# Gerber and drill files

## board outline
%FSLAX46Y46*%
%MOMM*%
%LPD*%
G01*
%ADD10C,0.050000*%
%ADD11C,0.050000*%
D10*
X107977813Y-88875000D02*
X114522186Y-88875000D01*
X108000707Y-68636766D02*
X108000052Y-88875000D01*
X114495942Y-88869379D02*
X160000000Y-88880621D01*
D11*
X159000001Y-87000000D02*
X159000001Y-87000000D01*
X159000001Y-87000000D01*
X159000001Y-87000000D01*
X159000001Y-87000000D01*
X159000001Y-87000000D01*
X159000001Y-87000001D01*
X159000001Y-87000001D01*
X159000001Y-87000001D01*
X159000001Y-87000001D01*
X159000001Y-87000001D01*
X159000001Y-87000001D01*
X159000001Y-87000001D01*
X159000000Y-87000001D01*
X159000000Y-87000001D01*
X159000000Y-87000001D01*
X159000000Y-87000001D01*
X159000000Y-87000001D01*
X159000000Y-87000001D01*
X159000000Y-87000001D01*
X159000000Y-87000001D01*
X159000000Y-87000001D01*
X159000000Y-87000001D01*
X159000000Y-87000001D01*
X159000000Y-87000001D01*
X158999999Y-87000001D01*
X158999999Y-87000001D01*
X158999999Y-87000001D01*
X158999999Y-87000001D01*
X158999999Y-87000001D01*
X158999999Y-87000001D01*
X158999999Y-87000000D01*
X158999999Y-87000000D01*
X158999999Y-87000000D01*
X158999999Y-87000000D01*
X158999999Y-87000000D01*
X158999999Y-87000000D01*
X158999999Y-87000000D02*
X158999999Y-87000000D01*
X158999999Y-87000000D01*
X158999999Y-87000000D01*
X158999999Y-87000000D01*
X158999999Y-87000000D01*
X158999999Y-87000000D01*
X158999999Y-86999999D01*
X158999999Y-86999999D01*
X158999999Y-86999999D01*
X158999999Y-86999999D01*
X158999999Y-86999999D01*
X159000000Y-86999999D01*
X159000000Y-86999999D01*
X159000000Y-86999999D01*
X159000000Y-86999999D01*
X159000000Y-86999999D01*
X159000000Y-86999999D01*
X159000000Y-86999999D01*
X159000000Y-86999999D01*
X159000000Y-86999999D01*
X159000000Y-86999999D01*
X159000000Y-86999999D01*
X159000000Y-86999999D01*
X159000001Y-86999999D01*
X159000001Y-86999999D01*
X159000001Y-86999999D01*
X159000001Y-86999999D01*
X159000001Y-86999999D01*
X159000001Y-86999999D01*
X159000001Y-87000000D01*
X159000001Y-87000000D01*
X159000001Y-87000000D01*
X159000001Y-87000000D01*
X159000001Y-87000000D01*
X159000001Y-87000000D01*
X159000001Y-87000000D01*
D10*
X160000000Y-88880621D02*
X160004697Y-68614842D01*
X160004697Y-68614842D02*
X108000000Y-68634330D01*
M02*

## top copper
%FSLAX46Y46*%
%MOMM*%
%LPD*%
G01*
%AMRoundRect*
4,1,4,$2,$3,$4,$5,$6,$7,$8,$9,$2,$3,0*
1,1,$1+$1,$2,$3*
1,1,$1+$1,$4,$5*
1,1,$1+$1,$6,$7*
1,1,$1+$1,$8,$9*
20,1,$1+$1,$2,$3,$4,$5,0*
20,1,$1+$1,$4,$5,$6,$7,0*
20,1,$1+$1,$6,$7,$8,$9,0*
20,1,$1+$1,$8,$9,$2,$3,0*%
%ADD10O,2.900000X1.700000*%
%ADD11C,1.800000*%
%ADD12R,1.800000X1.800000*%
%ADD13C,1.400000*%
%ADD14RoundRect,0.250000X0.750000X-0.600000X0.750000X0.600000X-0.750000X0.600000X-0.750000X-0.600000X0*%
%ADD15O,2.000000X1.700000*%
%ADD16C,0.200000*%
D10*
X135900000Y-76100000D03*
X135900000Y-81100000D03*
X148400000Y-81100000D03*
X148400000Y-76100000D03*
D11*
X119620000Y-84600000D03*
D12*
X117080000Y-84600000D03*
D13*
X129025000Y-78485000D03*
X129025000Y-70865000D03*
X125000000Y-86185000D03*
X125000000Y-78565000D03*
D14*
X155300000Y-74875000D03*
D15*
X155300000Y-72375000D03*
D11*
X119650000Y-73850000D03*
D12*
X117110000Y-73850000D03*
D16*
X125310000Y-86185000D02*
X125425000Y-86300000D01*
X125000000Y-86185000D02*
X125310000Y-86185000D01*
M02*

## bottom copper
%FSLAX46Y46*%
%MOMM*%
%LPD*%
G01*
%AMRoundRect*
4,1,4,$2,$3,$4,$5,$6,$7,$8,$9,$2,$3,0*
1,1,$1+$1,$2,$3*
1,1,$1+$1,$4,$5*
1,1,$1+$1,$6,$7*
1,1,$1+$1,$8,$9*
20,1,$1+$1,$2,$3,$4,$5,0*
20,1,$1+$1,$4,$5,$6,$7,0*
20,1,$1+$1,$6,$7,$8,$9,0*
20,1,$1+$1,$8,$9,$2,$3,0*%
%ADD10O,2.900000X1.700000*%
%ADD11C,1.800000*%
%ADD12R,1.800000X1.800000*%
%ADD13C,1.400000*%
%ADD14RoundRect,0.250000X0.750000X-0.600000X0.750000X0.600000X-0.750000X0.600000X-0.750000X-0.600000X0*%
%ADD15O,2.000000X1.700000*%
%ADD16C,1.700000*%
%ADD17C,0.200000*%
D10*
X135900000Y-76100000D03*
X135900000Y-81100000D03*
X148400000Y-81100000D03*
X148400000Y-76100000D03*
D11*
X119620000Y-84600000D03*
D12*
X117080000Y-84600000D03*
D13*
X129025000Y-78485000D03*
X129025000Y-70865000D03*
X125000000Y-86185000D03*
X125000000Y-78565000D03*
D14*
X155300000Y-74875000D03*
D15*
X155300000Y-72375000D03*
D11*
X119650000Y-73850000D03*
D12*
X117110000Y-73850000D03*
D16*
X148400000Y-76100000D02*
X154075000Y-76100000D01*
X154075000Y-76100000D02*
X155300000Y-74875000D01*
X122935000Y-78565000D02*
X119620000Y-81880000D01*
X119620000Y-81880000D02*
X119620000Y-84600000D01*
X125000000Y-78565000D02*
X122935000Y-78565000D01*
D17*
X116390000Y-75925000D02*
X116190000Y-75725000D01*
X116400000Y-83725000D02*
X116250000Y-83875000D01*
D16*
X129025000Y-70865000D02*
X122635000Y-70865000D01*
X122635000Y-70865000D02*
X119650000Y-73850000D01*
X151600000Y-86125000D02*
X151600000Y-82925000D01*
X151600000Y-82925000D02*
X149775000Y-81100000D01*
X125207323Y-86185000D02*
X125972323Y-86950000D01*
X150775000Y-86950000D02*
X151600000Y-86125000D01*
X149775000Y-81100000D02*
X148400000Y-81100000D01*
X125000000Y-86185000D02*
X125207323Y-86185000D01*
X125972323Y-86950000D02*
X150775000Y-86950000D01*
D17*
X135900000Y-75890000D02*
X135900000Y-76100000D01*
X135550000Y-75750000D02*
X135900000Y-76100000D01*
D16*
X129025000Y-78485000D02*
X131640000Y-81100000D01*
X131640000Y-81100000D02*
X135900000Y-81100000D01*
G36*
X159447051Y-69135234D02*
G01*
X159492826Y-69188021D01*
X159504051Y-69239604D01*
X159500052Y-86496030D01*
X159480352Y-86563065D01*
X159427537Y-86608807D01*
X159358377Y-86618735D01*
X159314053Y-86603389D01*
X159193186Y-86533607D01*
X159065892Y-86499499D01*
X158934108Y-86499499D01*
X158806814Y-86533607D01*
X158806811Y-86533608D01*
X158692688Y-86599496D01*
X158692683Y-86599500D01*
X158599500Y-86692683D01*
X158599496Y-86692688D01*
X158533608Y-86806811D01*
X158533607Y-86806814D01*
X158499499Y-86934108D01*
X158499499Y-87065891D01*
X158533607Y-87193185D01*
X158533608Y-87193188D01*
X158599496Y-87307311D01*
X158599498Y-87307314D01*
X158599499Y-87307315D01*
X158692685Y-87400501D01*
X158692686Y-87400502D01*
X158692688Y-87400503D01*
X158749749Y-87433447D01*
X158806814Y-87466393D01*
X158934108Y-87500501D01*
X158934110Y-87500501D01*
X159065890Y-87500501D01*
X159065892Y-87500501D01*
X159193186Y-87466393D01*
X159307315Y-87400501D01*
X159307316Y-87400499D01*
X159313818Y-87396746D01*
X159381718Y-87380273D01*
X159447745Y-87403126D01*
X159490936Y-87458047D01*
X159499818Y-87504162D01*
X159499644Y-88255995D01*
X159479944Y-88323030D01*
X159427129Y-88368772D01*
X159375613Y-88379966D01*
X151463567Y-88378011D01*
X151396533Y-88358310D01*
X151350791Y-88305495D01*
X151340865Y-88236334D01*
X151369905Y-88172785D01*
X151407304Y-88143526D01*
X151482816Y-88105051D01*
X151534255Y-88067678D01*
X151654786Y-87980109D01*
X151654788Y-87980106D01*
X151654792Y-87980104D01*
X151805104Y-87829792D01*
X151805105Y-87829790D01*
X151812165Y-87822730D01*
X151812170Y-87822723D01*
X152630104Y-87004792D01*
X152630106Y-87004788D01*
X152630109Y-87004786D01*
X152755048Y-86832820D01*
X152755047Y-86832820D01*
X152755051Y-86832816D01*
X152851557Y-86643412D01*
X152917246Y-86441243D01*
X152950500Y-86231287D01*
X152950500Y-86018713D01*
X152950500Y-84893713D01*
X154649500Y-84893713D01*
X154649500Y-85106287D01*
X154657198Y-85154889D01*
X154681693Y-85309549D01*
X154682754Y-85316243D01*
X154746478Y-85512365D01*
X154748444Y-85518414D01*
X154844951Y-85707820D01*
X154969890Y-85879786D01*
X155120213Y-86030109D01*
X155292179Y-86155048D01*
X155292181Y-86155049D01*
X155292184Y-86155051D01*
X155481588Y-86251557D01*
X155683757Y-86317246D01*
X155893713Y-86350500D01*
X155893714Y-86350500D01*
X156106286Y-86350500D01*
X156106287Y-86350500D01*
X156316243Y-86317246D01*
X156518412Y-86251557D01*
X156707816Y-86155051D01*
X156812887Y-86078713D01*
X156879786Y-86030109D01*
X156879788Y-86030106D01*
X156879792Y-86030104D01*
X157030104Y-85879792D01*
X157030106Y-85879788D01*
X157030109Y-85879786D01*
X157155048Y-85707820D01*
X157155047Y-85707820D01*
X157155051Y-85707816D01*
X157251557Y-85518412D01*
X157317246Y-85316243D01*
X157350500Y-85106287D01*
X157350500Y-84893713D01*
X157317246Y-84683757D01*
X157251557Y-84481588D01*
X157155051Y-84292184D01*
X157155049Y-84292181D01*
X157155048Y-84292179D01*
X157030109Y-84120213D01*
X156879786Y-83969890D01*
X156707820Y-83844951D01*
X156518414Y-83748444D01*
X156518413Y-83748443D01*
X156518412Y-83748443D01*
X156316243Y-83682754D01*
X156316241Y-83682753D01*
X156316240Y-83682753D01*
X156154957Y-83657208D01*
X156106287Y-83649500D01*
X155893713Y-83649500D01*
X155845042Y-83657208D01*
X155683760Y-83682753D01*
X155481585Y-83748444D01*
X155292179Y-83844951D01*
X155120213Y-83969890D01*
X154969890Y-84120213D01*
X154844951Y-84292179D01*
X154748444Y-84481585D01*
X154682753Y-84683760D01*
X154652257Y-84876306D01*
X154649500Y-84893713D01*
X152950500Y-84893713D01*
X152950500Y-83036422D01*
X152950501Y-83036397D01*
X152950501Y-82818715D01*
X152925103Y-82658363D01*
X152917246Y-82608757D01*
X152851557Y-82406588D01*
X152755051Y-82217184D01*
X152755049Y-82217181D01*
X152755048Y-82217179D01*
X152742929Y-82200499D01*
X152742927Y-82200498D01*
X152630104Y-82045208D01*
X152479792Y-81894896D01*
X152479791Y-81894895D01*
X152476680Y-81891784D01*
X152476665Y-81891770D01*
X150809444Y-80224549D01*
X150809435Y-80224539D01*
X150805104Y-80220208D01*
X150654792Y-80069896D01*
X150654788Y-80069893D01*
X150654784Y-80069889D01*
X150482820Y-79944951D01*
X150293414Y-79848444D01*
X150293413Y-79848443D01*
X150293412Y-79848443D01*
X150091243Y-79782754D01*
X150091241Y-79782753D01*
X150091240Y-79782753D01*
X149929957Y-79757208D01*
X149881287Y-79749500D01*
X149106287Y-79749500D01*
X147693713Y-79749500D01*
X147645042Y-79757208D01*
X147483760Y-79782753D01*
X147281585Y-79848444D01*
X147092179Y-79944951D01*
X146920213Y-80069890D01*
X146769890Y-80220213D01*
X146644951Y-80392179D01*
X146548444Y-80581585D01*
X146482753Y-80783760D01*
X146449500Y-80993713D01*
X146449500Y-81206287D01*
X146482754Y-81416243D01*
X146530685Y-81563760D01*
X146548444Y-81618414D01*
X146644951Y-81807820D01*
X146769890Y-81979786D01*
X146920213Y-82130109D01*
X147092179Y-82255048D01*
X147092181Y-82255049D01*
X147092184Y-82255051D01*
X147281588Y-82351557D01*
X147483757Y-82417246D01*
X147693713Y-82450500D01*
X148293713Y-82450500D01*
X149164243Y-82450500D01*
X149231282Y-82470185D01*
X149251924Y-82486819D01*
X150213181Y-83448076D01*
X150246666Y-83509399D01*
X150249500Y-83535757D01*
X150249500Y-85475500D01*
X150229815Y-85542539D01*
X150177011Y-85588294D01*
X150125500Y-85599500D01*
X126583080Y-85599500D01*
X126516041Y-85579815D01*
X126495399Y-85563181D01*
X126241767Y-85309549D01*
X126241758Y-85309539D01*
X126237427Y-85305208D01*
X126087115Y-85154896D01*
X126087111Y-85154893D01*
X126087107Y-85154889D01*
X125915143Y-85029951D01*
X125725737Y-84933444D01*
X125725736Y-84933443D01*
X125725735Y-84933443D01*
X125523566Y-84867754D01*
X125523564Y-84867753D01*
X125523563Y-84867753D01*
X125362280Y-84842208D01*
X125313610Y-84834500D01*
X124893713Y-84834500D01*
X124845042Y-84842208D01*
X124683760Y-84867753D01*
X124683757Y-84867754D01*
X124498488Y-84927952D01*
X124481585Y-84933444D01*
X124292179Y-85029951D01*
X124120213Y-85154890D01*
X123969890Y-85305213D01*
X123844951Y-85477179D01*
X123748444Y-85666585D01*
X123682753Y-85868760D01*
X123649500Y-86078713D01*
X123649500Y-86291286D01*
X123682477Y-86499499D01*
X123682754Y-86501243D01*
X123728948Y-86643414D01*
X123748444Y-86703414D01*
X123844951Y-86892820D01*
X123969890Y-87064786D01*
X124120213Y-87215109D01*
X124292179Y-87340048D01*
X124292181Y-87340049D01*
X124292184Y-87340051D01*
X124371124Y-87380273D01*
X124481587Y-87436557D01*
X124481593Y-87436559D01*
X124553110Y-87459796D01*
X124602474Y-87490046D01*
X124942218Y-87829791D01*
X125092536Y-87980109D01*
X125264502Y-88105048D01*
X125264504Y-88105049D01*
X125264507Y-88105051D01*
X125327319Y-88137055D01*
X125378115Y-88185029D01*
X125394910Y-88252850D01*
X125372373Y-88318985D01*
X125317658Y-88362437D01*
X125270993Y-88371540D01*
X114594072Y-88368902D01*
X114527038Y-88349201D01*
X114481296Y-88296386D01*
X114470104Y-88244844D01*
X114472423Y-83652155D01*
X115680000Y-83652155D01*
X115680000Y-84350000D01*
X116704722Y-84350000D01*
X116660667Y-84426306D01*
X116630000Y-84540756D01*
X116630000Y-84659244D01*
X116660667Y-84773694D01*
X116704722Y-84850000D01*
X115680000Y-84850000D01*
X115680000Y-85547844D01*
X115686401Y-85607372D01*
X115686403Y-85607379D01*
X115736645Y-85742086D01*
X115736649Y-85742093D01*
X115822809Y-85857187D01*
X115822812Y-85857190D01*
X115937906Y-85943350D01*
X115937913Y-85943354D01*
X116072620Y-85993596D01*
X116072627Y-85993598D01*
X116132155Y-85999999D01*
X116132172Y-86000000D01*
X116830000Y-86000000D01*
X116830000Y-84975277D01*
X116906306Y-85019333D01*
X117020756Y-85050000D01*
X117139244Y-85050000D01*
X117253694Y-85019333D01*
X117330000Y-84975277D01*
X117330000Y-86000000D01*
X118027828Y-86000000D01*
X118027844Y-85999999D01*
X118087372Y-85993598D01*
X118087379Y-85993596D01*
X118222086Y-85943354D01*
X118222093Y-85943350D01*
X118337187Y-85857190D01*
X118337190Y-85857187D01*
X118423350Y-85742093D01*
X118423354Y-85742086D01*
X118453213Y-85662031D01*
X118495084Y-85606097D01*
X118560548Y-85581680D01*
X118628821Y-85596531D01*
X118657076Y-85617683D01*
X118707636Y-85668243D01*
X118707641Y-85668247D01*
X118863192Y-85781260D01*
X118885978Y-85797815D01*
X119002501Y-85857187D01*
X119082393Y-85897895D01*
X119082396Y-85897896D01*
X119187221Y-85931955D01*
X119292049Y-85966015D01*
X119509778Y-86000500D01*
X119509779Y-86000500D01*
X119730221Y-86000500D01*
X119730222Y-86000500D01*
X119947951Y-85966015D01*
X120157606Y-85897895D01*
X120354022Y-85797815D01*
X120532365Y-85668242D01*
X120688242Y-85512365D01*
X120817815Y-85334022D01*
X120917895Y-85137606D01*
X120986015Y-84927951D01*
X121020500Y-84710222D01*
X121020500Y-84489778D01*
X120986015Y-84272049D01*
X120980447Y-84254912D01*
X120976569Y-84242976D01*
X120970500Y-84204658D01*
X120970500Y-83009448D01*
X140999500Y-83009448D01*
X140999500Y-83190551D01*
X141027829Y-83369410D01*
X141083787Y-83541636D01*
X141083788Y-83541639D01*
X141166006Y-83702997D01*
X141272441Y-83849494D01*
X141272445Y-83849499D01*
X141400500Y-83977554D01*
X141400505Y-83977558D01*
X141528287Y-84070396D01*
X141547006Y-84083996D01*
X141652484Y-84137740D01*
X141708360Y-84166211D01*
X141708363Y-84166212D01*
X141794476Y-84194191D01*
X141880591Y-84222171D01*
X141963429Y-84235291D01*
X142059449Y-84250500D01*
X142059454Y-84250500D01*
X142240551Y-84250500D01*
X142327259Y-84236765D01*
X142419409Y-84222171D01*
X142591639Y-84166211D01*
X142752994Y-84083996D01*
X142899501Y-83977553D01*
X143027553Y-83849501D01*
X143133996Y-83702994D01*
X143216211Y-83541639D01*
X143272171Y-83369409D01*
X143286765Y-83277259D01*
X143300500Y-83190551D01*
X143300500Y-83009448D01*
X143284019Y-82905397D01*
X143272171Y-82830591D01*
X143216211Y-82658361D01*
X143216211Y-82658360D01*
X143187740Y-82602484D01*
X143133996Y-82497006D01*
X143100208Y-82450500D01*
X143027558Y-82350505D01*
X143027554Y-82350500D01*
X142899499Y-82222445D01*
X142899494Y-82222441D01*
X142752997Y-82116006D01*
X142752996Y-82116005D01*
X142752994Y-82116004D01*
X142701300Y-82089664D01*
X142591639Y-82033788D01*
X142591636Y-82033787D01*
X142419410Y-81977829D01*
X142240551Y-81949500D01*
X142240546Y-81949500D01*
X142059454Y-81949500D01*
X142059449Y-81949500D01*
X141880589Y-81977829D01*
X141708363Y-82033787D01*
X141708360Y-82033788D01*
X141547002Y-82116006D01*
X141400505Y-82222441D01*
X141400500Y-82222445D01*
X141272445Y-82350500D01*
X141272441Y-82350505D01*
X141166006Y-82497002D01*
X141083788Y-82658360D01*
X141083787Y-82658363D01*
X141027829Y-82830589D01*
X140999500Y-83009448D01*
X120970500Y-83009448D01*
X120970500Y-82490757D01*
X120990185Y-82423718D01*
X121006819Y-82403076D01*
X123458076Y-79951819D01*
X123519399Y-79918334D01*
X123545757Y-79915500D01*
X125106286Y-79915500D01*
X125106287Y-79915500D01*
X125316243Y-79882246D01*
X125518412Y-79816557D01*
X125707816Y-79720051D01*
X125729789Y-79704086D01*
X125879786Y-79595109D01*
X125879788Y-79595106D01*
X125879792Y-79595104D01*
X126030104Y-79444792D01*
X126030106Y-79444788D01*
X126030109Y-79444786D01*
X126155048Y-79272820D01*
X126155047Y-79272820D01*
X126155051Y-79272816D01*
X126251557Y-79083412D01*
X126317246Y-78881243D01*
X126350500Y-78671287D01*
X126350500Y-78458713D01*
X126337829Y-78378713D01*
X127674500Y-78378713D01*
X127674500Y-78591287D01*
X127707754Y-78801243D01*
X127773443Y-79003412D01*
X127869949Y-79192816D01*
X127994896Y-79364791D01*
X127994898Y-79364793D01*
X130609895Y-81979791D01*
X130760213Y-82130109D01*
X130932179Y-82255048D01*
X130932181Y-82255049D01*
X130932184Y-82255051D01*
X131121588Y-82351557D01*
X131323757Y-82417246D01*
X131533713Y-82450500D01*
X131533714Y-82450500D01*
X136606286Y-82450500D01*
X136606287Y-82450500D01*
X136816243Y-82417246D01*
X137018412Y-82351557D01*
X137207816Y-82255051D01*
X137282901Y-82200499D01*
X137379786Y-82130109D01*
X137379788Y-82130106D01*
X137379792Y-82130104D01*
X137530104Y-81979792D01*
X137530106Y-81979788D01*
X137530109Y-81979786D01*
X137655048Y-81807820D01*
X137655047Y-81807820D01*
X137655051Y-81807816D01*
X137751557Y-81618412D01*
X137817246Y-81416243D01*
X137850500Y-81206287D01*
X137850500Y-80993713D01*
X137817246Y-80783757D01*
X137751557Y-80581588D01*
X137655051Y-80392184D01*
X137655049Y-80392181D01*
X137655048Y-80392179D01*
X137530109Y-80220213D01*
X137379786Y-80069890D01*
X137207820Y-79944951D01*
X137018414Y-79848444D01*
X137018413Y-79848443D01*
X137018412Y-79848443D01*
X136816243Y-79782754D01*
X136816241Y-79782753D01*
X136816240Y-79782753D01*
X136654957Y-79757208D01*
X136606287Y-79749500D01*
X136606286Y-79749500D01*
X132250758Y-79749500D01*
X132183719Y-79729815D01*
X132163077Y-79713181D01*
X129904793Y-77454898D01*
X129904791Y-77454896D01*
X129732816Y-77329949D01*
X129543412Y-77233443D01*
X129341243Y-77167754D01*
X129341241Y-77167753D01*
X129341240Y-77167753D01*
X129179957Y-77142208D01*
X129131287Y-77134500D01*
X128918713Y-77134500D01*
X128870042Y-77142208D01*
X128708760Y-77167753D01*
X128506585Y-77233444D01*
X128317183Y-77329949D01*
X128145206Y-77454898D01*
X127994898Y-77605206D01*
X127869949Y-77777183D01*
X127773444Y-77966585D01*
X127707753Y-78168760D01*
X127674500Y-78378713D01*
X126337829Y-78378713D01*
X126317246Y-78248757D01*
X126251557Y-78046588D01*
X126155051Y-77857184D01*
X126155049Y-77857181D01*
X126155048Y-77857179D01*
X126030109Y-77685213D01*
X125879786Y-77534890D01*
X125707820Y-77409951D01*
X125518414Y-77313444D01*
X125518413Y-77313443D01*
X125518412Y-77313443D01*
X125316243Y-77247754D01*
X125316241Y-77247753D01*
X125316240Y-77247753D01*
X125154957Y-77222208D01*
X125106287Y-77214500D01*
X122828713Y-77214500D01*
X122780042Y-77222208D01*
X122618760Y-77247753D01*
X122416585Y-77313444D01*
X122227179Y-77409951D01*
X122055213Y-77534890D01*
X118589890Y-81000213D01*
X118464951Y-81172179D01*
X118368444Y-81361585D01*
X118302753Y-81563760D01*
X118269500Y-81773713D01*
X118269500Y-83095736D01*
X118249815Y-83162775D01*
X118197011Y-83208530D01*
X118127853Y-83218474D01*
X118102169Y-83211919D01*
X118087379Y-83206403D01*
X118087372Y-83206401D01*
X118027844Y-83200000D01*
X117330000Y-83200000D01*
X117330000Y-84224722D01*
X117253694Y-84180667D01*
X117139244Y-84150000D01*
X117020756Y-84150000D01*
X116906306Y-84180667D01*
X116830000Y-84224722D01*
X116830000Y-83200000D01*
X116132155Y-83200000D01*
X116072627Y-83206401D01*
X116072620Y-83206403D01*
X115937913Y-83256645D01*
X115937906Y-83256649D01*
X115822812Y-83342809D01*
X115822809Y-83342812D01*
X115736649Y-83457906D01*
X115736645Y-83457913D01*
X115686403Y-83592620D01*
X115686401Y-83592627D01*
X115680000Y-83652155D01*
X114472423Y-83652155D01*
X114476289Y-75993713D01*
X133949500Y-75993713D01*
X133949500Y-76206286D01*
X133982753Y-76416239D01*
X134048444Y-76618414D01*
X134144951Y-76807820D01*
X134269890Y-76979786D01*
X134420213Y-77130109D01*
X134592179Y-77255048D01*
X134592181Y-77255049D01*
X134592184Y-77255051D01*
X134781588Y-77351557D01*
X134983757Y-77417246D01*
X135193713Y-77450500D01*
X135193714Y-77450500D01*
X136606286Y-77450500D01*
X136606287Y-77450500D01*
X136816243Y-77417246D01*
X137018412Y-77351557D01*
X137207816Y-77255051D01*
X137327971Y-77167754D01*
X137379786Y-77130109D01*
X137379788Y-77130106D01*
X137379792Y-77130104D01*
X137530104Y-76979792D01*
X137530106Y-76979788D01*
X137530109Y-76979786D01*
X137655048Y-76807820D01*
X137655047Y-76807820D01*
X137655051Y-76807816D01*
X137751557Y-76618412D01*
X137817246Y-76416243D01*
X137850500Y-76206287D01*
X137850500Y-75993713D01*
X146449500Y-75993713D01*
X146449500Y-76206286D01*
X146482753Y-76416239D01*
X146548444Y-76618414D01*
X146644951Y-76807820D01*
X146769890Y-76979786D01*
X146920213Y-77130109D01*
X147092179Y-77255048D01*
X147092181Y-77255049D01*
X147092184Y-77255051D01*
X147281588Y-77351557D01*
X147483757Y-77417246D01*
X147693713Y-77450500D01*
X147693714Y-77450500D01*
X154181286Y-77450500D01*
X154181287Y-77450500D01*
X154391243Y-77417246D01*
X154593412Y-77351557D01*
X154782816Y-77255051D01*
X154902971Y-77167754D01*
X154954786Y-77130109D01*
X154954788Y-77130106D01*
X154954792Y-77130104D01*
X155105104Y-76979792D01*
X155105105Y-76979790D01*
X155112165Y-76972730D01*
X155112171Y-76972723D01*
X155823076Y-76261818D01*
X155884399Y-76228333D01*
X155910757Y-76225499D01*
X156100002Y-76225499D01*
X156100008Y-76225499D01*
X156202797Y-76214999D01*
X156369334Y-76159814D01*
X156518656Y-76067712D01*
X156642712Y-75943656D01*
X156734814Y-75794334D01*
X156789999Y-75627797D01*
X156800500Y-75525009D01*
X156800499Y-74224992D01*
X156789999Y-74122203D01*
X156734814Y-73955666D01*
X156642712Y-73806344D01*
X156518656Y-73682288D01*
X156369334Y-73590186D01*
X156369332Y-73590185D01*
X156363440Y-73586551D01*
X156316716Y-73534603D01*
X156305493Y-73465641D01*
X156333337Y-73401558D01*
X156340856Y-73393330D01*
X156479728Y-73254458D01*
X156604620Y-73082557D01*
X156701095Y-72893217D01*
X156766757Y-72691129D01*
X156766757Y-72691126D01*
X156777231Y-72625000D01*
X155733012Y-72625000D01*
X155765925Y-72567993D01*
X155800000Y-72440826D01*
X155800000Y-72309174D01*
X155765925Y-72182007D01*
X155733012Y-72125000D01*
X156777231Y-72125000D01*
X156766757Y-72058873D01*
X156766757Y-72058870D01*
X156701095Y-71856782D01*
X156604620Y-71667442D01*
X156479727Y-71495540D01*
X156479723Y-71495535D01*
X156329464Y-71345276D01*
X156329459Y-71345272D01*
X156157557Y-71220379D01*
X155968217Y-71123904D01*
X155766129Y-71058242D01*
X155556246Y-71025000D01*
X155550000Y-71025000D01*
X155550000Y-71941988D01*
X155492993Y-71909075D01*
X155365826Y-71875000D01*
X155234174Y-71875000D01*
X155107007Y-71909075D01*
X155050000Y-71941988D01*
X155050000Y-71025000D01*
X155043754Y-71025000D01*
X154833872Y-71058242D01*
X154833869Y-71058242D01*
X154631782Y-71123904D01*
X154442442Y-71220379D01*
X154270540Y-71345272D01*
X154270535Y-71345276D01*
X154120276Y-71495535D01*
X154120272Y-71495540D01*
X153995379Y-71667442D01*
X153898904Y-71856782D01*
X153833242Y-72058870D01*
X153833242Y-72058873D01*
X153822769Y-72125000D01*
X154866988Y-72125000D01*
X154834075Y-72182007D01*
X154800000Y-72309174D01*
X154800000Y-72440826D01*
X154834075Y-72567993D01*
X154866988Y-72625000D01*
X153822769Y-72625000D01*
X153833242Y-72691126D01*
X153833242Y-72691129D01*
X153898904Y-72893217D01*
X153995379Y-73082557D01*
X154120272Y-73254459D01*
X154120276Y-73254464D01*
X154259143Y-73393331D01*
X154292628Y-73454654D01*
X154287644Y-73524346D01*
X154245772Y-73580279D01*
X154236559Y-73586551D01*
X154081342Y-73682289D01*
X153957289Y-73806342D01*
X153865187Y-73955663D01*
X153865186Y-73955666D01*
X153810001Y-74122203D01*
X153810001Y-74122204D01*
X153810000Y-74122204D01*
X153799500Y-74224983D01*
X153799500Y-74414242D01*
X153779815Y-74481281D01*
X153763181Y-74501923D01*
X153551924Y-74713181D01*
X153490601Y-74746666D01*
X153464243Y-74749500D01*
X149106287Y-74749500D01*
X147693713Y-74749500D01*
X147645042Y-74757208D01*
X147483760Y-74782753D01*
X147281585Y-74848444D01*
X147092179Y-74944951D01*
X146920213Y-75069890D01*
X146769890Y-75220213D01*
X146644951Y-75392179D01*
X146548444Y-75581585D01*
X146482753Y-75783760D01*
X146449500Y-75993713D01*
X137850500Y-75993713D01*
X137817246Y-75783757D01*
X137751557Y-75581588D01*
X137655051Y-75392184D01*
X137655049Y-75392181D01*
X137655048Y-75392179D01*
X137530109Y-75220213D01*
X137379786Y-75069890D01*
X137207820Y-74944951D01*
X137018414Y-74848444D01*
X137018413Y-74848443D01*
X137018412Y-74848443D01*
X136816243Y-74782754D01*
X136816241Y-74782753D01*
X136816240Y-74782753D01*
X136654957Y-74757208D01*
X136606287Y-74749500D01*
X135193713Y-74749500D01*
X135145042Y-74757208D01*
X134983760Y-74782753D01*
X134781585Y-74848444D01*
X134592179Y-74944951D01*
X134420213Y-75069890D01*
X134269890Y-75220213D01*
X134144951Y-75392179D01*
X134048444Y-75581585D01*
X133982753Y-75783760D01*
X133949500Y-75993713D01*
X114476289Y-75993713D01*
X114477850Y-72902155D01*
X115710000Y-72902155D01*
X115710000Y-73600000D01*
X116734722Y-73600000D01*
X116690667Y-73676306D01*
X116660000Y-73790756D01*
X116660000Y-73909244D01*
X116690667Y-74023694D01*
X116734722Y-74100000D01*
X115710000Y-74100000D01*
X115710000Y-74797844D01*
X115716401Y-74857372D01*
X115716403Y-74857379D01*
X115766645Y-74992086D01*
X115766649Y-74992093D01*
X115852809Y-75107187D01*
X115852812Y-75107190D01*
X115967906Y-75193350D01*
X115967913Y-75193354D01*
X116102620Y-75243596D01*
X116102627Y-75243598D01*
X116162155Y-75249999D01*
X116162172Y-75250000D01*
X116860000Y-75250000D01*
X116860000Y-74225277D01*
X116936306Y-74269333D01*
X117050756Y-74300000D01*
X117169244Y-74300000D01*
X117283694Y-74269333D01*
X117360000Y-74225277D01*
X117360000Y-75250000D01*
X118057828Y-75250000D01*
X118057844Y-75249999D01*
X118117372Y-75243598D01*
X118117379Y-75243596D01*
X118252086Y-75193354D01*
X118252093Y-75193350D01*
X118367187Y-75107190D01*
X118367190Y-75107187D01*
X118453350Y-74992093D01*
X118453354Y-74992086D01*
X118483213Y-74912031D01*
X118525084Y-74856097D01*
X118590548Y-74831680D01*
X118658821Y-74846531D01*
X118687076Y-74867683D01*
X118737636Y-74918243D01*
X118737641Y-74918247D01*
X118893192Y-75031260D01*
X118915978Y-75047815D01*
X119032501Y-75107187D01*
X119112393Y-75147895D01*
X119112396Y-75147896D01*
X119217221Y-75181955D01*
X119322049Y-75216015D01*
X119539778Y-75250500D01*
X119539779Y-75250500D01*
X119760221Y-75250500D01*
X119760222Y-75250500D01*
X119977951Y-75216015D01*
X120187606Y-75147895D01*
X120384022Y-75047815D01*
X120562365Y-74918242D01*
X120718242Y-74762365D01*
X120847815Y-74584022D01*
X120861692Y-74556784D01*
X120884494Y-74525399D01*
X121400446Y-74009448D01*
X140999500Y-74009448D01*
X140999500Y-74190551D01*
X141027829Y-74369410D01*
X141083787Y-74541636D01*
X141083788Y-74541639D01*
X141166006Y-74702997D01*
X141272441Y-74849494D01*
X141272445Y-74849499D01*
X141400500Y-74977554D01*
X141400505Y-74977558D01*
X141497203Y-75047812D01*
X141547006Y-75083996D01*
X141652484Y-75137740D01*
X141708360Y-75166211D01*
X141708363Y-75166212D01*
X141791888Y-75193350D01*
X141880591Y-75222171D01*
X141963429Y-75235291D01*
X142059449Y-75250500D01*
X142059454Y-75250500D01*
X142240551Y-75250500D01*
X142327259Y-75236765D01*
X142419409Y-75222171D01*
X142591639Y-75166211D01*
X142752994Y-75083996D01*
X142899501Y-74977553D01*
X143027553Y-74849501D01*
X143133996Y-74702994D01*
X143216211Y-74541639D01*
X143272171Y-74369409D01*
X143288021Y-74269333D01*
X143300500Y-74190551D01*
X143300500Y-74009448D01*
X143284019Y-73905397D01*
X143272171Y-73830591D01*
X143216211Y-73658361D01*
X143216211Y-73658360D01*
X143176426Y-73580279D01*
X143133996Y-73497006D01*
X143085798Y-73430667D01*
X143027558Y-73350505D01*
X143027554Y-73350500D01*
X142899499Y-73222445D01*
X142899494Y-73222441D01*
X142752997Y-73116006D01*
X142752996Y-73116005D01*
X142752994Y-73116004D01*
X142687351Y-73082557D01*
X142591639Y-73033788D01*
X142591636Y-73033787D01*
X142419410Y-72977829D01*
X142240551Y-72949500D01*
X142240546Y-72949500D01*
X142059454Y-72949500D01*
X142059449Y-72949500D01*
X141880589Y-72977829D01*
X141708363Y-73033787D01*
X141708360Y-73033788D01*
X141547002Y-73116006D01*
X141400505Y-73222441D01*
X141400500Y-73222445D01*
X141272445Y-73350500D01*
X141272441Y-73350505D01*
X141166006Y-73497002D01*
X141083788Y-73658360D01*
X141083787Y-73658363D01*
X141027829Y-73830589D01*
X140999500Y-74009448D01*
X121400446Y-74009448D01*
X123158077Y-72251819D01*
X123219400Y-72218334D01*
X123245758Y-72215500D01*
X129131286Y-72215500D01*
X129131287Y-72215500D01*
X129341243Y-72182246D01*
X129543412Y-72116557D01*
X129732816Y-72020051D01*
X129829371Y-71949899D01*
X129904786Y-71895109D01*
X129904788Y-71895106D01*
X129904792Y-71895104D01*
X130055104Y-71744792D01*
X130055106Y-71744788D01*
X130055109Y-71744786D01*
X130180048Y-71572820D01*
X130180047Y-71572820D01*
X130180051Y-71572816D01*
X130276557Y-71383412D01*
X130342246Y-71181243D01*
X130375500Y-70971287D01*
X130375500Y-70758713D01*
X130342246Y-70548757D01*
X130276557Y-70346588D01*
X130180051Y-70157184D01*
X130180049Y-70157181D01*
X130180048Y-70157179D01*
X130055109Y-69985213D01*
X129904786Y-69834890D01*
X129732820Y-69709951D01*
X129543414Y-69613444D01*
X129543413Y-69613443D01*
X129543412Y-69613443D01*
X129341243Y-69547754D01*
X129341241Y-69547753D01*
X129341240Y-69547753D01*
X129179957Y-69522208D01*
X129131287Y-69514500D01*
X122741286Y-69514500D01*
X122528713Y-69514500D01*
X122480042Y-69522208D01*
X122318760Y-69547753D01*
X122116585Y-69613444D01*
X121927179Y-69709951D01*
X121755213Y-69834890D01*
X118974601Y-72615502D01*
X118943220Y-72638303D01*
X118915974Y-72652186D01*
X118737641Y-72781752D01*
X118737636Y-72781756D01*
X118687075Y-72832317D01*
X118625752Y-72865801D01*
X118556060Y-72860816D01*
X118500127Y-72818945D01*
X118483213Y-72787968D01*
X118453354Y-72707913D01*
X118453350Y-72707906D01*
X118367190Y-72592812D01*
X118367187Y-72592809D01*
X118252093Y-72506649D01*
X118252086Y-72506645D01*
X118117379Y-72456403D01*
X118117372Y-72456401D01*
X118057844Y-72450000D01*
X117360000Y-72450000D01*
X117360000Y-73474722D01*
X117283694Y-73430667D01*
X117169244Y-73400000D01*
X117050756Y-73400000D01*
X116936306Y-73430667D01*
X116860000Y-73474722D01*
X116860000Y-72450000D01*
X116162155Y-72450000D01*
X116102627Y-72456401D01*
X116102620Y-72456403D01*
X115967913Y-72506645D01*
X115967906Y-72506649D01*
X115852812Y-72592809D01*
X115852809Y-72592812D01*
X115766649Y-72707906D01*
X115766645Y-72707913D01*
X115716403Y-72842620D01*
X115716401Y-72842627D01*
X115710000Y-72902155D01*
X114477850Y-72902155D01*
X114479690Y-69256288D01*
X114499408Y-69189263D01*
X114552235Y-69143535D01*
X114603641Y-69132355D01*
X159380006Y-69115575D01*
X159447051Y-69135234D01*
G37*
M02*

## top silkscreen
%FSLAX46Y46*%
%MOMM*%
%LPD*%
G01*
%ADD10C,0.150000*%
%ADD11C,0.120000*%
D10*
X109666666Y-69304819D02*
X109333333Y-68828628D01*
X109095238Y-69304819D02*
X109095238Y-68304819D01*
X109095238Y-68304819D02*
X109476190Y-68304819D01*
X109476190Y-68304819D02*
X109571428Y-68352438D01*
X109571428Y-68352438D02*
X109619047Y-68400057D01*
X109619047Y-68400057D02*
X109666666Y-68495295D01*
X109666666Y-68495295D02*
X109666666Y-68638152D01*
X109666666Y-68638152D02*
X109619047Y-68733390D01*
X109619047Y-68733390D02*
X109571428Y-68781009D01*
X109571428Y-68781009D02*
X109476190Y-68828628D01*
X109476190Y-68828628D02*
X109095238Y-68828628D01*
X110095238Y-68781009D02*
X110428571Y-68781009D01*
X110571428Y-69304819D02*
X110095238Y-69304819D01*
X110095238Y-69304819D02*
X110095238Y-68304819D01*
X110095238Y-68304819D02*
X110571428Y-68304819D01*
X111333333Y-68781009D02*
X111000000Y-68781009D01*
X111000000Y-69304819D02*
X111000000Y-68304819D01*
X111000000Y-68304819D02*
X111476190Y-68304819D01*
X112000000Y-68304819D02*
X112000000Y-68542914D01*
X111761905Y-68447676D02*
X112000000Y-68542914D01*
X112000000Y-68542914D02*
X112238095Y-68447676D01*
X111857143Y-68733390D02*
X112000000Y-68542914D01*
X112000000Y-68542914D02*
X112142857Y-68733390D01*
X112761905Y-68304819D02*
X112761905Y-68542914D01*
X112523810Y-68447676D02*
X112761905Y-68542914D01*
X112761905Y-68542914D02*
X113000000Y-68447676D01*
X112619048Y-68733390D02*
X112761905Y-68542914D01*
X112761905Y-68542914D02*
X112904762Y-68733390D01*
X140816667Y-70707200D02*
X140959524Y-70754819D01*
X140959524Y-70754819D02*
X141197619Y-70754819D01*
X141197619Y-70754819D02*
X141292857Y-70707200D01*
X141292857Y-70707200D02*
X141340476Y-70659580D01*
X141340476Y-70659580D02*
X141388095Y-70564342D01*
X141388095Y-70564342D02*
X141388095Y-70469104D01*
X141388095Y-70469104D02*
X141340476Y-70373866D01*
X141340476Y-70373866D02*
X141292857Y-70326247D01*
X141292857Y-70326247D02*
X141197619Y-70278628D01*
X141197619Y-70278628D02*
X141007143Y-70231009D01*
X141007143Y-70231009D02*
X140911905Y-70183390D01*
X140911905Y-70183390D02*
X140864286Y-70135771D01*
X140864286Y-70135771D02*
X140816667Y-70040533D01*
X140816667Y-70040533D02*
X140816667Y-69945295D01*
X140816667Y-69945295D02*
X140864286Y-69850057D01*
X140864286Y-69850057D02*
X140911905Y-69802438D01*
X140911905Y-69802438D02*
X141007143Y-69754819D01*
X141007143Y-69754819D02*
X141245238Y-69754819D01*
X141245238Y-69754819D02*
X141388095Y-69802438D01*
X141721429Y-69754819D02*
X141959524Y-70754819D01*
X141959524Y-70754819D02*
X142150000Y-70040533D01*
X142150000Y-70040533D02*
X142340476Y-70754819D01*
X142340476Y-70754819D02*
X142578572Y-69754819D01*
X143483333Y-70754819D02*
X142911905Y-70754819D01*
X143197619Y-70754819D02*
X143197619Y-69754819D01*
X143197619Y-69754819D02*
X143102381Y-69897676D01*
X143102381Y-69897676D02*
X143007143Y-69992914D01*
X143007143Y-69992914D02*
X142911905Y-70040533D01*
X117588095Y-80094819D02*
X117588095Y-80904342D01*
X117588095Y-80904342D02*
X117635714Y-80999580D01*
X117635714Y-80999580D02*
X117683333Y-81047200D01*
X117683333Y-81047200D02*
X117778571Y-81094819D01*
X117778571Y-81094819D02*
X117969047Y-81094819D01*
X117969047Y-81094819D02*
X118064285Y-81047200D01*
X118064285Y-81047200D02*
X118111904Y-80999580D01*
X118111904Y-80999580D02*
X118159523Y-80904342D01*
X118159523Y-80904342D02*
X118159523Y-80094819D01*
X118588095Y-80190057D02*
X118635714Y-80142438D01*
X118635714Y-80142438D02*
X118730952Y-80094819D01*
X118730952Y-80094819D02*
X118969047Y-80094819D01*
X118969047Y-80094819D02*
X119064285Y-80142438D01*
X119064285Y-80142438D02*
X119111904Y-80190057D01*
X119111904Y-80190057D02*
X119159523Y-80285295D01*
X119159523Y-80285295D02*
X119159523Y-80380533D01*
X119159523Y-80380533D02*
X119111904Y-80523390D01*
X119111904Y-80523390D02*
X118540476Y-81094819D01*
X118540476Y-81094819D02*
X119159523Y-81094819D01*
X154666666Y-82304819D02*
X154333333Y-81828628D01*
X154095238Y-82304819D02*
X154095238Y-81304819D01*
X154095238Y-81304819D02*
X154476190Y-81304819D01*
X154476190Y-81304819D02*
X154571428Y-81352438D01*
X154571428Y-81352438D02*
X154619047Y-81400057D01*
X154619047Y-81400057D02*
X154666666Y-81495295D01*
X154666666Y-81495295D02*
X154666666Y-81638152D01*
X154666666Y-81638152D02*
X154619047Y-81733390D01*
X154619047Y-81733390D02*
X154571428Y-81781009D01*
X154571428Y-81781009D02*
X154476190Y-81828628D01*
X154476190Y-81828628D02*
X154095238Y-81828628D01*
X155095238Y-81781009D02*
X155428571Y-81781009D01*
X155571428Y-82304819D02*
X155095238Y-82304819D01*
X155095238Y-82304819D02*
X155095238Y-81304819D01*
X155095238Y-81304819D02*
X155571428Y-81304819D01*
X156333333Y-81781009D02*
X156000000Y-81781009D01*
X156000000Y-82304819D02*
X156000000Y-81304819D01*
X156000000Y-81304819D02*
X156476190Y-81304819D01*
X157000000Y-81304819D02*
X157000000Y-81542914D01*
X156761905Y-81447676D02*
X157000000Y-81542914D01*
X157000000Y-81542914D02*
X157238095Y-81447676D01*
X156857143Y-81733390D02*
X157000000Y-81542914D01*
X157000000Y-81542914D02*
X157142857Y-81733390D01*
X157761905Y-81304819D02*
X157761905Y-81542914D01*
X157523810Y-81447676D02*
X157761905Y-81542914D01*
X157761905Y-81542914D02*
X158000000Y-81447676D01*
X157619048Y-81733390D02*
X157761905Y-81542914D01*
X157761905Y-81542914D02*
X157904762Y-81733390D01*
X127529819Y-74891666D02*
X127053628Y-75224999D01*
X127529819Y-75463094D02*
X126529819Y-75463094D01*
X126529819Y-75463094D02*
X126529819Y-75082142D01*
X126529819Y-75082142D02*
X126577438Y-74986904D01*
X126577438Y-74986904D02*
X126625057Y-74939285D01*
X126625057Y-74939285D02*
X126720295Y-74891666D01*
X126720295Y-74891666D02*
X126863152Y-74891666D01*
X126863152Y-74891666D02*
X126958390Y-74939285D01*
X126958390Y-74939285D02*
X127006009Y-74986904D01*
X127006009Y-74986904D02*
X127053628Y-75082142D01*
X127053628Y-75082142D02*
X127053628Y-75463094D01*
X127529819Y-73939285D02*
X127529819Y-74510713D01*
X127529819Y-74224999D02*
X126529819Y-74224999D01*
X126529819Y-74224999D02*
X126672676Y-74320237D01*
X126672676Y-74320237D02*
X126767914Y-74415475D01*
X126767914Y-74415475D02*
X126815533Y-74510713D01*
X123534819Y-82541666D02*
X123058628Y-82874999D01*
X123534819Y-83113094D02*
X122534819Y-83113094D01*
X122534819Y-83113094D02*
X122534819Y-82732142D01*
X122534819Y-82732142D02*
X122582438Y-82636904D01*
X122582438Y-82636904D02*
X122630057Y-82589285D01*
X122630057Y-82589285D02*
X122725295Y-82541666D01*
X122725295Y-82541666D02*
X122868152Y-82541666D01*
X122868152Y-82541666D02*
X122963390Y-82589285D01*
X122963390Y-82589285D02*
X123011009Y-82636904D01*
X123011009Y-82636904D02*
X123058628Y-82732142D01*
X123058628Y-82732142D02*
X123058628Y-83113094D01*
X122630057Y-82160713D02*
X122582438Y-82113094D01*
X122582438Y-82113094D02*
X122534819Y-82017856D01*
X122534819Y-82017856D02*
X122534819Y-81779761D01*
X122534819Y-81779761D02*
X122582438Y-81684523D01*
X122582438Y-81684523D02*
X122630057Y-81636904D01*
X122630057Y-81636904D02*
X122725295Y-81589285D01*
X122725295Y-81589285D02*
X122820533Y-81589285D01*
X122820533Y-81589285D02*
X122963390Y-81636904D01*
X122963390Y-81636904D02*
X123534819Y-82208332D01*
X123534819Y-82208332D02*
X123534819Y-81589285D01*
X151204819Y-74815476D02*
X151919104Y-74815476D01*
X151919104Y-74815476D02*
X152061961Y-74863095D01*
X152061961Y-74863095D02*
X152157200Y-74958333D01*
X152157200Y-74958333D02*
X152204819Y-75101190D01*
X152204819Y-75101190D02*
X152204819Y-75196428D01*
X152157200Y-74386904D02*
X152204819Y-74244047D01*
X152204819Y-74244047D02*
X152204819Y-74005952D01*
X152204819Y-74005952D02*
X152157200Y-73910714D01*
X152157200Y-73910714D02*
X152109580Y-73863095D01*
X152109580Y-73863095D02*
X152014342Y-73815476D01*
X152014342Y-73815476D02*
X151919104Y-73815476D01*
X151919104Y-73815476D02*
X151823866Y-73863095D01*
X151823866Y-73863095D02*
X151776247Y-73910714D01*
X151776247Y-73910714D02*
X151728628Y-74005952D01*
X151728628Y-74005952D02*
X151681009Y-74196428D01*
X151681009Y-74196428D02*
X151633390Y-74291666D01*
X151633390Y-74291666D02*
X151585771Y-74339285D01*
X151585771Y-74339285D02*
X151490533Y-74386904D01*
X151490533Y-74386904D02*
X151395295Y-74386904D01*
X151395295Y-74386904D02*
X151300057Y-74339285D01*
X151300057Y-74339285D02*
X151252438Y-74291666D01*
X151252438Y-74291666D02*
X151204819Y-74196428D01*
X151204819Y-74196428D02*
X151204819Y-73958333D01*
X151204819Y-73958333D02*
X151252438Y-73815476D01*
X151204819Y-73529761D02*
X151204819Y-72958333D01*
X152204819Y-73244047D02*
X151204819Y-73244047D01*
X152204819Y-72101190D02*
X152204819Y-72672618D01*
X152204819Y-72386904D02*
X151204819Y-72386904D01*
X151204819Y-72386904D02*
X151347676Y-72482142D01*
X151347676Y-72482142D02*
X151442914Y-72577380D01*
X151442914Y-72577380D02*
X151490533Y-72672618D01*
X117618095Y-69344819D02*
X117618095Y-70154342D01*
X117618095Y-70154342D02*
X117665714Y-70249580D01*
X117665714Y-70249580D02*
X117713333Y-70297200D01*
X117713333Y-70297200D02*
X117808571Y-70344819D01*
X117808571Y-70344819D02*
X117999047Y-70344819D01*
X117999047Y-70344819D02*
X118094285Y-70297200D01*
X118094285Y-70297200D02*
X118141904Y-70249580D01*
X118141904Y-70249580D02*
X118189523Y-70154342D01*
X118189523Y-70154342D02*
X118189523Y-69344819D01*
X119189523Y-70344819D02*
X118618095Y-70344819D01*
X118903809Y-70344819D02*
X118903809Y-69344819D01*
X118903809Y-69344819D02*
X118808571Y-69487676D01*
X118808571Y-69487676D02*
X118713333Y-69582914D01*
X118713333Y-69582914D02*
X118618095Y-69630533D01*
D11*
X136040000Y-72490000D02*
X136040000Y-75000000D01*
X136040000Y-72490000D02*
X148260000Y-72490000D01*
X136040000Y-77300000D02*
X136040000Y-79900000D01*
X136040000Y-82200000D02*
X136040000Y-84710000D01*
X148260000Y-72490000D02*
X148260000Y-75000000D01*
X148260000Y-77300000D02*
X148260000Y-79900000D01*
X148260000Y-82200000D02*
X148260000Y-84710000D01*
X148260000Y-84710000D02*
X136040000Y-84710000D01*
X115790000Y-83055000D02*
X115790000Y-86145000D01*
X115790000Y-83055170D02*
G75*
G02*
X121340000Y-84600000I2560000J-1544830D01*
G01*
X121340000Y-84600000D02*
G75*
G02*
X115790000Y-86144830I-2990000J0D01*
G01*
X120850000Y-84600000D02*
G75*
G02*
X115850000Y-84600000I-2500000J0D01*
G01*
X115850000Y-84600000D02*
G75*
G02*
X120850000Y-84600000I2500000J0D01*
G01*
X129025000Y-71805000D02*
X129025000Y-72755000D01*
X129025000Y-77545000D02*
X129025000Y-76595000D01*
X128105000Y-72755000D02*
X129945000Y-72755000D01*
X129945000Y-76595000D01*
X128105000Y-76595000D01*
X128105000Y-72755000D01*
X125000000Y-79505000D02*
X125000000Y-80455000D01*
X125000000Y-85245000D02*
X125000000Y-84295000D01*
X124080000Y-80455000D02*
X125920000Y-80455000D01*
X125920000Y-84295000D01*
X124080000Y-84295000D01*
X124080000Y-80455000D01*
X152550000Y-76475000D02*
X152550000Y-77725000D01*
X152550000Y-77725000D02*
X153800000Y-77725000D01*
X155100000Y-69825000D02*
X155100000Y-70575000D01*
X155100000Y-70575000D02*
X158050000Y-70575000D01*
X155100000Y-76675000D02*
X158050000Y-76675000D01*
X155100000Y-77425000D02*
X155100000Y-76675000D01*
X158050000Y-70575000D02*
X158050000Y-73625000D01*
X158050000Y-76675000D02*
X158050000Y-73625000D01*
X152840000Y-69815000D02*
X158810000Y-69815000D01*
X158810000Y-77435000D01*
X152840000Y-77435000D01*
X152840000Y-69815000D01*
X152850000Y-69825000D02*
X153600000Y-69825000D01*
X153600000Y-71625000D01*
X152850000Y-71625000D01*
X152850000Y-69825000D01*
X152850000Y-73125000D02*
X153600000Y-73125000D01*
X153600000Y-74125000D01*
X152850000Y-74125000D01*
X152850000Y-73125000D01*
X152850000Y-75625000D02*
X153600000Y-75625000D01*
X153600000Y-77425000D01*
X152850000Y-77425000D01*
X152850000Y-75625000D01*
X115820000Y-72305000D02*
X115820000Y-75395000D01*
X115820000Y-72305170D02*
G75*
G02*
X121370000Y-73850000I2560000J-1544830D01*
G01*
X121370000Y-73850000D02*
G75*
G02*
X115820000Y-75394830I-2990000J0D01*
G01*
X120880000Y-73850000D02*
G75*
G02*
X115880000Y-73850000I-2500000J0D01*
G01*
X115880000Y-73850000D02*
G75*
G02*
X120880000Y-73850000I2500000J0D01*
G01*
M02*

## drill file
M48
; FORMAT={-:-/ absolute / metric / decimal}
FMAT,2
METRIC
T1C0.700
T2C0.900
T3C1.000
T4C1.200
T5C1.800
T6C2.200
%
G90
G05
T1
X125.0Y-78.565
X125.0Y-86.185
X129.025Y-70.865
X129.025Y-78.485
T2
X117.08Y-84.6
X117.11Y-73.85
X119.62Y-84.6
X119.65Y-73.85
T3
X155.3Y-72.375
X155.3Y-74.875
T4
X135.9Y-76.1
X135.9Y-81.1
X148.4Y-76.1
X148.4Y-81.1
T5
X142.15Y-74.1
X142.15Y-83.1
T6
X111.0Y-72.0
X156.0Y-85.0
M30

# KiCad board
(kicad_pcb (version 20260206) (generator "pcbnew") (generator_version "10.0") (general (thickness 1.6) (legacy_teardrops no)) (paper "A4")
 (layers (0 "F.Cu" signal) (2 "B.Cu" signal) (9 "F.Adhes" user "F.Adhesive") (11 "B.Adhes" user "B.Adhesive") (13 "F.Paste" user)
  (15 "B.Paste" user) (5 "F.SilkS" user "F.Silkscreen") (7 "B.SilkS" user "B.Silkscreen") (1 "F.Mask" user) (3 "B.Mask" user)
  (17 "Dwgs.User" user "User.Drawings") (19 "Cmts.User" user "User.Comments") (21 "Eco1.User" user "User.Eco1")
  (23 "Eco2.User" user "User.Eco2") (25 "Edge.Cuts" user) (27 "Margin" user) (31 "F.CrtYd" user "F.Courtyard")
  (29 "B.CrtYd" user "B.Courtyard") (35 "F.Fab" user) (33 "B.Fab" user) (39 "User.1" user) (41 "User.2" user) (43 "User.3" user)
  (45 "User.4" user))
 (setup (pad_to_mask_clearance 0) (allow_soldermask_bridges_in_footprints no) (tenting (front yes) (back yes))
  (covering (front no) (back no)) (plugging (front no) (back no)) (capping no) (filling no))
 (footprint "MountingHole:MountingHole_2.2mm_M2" (layer "F.Cu") (at 111 72)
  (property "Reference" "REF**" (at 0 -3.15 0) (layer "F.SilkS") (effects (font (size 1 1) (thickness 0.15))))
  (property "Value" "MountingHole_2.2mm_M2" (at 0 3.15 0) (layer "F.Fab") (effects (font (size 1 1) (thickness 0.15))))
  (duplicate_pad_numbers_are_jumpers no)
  (pad "" np_thru_hole circle (at 0 0) (size 2.2 2.2) (drill 2.2) (layers "*.Cu" "*.Mask")))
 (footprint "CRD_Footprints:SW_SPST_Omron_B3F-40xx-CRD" (layer "F.Cu") (at 135.9 76.1)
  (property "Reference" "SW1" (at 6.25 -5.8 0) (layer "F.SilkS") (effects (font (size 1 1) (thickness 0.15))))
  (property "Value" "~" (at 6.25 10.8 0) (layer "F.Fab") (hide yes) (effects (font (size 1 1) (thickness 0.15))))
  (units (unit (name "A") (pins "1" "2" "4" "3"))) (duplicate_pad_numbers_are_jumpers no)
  (fp_line (start 0.14 -3.61) (end 0.14 -1.1) (stroke (width 0.12) (type default)) (layer "F.SilkS"))
  (fp_line (start 0.14 -3.61) (end 12.36 -3.61) (stroke (width 0.12) (type default)) (layer "F.SilkS"))
  (fp_line (start 0.14 1.2) (end 0.14 3.8) (stroke (width 0.12) (type default)) (layer "F.SilkS"))
  (fp_line (start 0.14 6.1) (end 0.14 8.61) (stroke (width 0.12) (type default)) (layer "F.SilkS"))
  (fp_line (start 12.36 -3.61) (end 12.36 -1.1) (stroke (width 0.12) (type default)) (layer "F.SilkS"))
  (fp_line (start 12.36 1.2) (end 12.36 3.8) (stroke (width 0.12) (type default)) (layer "F.SilkS"))
  (fp_line (start 12.36 6.1) (end 12.36 8.61) (stroke (width 0.12) (type default)) (layer "F.SilkS"))
  (fp_line (start 12.36 8.61) (end 0.14 8.61) (stroke (width 0.12) (type default)) (layer "F.SilkS"))
  (pad "" np_thru_hole circle (at 6.25 -2) (size 1.8 1.8) (drill 1.8) (layers "*.Cu" "*.Mask"))
  (pad "" np_thru_hole circle (at 6.25 7) (size 1.8 1.8) (drill 1.8) (layers "*.Cu" "*.Mask"))
  (pad "1" thru_hole oval (at 0 0) (size 2.9 1.7) (drill 1.2) (layers "*.Cu" "*.Mask") (remove_unused_layers no)
   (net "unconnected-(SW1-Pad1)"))
  (pad "2" thru_hole oval (at 0 5) (size 2.9 1.7) (drill 1.2) (layers "*.Cu" "*.Mask") (remove_unused_layers no) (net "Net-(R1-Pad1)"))
  (pad "3" thru_hole oval (at 12.5 5) (size 2.9 1.7) (drill 1.2) (layers "*.Cu" "*.Mask") (remove_unused_layers no) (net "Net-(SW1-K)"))
  (pad "4" thru_hole oval (at 12.5 0) (size 2.9 1.7) (drill 1.2) (layers "*.Cu" "*.Mask") (remove_unused_layers no) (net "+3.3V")))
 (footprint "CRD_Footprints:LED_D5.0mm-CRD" (layer "F.Cu") (at 117.08 84.6)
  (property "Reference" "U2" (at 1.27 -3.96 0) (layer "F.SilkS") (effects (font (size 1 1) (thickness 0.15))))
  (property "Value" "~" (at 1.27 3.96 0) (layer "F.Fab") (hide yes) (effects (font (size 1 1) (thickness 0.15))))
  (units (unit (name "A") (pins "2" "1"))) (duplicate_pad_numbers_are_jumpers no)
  (fp_line (start -1.29 -1.545) (end -1.29 1.545) (stroke (width 0.12) (type solid)) (layer "F.SilkS"))
  (fp_arc (start -1.29 -1.54483) (mid 2.071779 -2.880495) (end 4.26 0) (stroke (width 0.12) (type solid)) (layer "F.SilkS"))
  (fp_arc (start 4.26 0) (mid 2.071779 2.880495) (end -1.29 1.54483) (stroke (width 0.12) (type solid)) (layer "F.SilkS"))
  (fp_circle (center 1.27 0) (end 3.77 0) (stroke (width 0.12) (type solid)) (fill no) (layer "F.SilkS"))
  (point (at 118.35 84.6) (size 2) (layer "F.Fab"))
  (pad "1" thru_hole circle (at 2.54 0) (size 1.8 1.8) (drill 0.9) (layers "*.Cu" "*.Mask") (remove_unused_layers no) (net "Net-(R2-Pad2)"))
  (pad "2" thru_hole rect (at 0 0) (size 1.8 1.8) (drill 0.9) (layers "*.Cu" "*.Mask") (remove_unused_layers no) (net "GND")))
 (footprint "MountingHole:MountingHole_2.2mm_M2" (layer "F.Cu") (at 156 85)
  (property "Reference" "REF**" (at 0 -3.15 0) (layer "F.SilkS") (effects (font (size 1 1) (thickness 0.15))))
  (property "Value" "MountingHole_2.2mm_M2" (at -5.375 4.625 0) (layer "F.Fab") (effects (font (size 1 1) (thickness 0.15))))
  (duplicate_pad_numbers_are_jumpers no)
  (pad "" np_thru_hole circle (at 0 0) (size 2.2 2.2) (drill 2.2) (layers "*.Cu" "*.Mask")))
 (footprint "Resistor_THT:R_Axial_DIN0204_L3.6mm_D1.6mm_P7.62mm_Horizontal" (layer "F.Cu") (at 129.025 78.485 90)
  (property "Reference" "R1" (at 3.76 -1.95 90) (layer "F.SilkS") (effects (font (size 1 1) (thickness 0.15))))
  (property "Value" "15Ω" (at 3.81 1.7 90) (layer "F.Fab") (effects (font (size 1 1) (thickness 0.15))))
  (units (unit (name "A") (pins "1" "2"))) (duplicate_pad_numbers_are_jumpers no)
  (fp_line (start 6.68 0) (end 5.73 0) (stroke (width 0.12) (type solid)) (layer "F.SilkS"))
  (fp_line (start 0.94 0) (end 1.89 0) (stroke (width 0.12) (type solid)) (layer "F.SilkS"))
  (fp_rect (start 1.89 -0.92) (end 5.73 0.92) (stroke (width 0.12) (type solid)) (fill no) (layer "F.SilkS"))
  (pad "1" thru_hole circle (at 0 0 90) (size 1.4 1.4) (drill 0.7) (layers "*.Cu" "*.Mask") (remove_unused_layers no) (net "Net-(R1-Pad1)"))
  (pad "2" thru_hole circle (at 7.62 0 90) (size 1.4 1.4) (drill 0.7) (layers "*.Cu" "*.Mask") (remove_unused_layers no)
   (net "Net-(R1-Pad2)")))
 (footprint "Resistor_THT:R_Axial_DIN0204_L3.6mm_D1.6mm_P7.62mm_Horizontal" (layer "F.Cu") (at 125 86.185 90)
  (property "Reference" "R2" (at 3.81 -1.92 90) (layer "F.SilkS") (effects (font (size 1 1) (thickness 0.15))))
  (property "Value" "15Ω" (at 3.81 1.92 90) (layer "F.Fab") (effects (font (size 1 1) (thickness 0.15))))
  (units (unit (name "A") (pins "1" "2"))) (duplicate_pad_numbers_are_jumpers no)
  (fp_line (start 6.68 0) (end 5.73 0) (stroke (width 0.12) (type solid)) (layer "F.SilkS"))
  (fp_line (start 0.94 0) (end 1.89 0) (stroke (width 0.12) (type solid)) (layer "F.SilkS"))
  (fp_rect (start 1.89 -0.92) (end 5.73 0.92) (stroke (width 0.12) (type solid)) (fill no) (layer "F.SilkS"))
  (pad "1" thru_hole circle (at 0 0 90) (size 1.4 1.4) (drill 0.7) (layers "*.Cu" "*.Mask") (remove_unused_layers no) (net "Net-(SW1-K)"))
  (pad "2" thru_hole circle (at 7.62 0 90) (size 1.4 1.4) (drill 0.7) (layers "*.Cu" "*.Mask") (remove_unused_layers no)
   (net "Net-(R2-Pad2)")))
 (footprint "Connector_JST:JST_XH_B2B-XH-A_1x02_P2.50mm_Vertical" (layer "F.Cu") (at 155.3 74.875 90)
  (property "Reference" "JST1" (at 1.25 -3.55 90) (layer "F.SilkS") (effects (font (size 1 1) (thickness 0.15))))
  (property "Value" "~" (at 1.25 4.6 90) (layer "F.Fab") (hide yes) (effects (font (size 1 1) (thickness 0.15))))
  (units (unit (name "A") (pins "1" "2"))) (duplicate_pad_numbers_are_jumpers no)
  (fp_line (start -1.6 -2.75) (end -2.85 -2.75) (stroke (width 0.12) (type solid)) (layer "F.SilkS"))
  (fp_line (start -2.85 -2.75) (end -2.85 -1.5) (stroke (width 0.12) (type solid)) (layer "F.SilkS"))
  (fp_line (start 5.05 -0.2) (end 4.3 -0.2) (stroke (width 0.12) (type solid)) (layer "F.SilkS"))
  (fp_line (start 4.3 -0.2) (end 4.3 2.75) (stroke (width 0.12) (type solid)) (layer "F.SilkS"))
  (fp_line (start -1.8 -0.2) (end -1.8 2.75) (stroke (width 0.12) (type solid)) (layer "F.SilkS"))
  (fp_line (start -2.55 -0.2) (end -1.8 -0.2) (stroke (width 0.12) (type solid)) (layer "F.SilkS"))
  (fp_line (start 4.3 2.75) (end 1.25 2.75) (stroke (width 0.12) (type solid)) (layer "F.SilkS"))
  (fp_line (start -1.8 2.75) (end 1.25 2.75) (stroke (width 0.12) (type solid)) (layer "F.SilkS"))
  (fp_rect (start -2.56 -2.46) (end 5.06 3.51) (stroke (width 0.12) (type solid)) (fill no) (layer "F.SilkS"))
  (fp_rect (start 3.25 -2.45) (end 5.05 -1.7) (stroke (width 0.12) (type solid)) (fill no) (layer "F.SilkS"))
  (fp_rect (start 0.75 -2.45) (end 1.75 -1.7) (stroke (width 0.12) (type solid)) (fill no) (layer "F.SilkS"))
  (fp_rect (start -2.55 -2.45) (end -0.75 -1.7) (stroke (width 0.12) (type solid)) (fill no) (layer "F.SilkS"))
  (pad "1" thru_hole roundrect (at 0 0 90) (size 1.7 2) (drill 1) (layers "*.Cu" "*.Mask") (remove_unused_layers no)
   (roundrect_rratio 0.147059) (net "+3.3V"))
  (pad "2" thru_hole oval (at 2.5 0 90) (size 1.7 2) (drill 1) (layers "*.Cu" "*.Mask") (remove_unused_layers no) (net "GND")))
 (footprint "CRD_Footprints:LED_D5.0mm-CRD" (layer "F.Cu") (at 117.11 73.85)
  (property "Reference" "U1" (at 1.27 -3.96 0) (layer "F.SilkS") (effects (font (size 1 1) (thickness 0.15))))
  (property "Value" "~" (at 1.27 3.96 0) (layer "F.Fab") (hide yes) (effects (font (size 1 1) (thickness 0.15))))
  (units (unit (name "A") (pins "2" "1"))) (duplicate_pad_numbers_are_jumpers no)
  (fp_line (start -1.29 -1.545) (end -1.29 1.545) (stroke (width 0.12) (type solid)) (layer "F.SilkS"))
  (fp_arc (start -1.29 -1.54483) (mid 2.071779 -2.880495) (end 4.26 0) (stroke (width 0.12) (type solid)) (layer "F.SilkS"))
  (fp_arc (start 4.26 0) (mid 2.071779 2.880495) (end -1.29 1.54483) (stroke (width 0.12) (type solid)) (layer "F.SilkS"))
  (fp_circle (center 1.27 0) (end 3.77 0) (stroke (width 0.12) (type solid)) (fill no) (layer "F.SilkS"))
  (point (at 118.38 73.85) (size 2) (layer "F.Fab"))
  (pad "1" thru_hole circle (at 2.54 0) (size 1.8 1.8) (drill 0.9) (layers "*.Cu" "*.Mask") (remove_unused_layers no) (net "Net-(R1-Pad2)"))
  (pad "2" thru_hole rect (at 0 0) (size 1.8 1.8) (drill 0.9) (layers "*.Cu" "*.Mask") (remove_unused_layers no) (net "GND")))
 (gr_line (start 107.977813 88.875) (end 114.522186 88.875) (stroke (width 0.05) (type default)) (layer "Edge.Cuts"))
 (gr_line (start 108.000707 68.636766) (end 108.000052 88.875) (stroke (width 0.05) (type default)) (layer "Edge.Cuts"))
 (gr_line (start 114.495942 88.869379) (end 160 88.880621) (stroke (width 0.05) (type default)) (layer "Edge.Cuts"))
 (gr_circle (center 159 87) (end 159 87) (stroke (width 0.05) (type default)) (fill no) (layer "Edge.Cuts"))
 (gr_line (start 160 88.880621) (end 160.004697 68.614842) (stroke (width 0.05) (type default)) (layer "Edge.Cuts"))
 (gr_line (start 160.004697 68.614842) (end 108 68.63433) (stroke (width 0.05) (type default)) (layer "Edge.Cuts"))
 (segment (start 148.4 76.1) (end 154.075 76.1) (width 1.7) (layer "B.Cu") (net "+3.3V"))
 (segment (start 154.075 76.1) (end 155.3 74.875) (width 1.7) (layer "B.Cu") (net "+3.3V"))
 (segment (start 122.935 78.565) (end 119.62 81.88) (width 1.7) (layer "B.Cu") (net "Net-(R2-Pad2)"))
 (segment (start 119.62 81.88) (end 119.62 84.6) (width 1.7) (layer "B.Cu") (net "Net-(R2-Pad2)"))
 (segment (start 125 78.565) (end 122.935 78.565) (width 1.7) (layer "B.Cu") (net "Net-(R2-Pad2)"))
 (segment (start 116.39 75.925) (end 116.19 75.725) (width 0.2) (layer "B.Cu") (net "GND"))
 (segment (start 116.4 83.725) (end 116.25 83.875) (width 0.2) (layer "B.Cu") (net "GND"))
 (segment (start 129.025 70.865) (end 122.635 70.865) (width 1.7) (layer "B.Cu") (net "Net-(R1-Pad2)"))
 (segment (start 122.635 70.865) (end 119.65 73.85) (width 1.7) (layer "B.Cu") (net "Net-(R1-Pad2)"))
 (segment (start 125.31 86.185) (end 125.425 86.3) (width 0.2) (layer "F.Cu") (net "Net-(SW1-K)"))
 (segment (start 125 86.185) (end 125.31 86.185) (width 0.2) (layer "F.Cu") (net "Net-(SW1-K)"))
 (segment (start 151.6 86.125) (end 151.6 82.925) (width 1.7) (layer "B.Cu") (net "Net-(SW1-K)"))
 (segment (start 151.6 82.925) (end 149.775 81.1) (width 1.7) (layer "B.Cu") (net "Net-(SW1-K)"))
 (segment (start 125.207323 86.185) (end 125.972323 86.95) (width 1.7) (layer "B.Cu") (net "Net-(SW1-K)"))
 (segment (start 150.775 86.95) (end 151.6 86.125) (width 1.7) (layer "B.Cu") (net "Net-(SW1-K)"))
 (segment (start 149.775 81.1) (end 148.4 81.1) (width 1.7) (layer "B.Cu") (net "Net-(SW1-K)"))
 (segment (start 125 86.185) (end 125.207323 86.185) (width 1.7) (layer "B.Cu") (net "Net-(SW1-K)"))
 (segment (start 125.972323 86.95) (end 150.775 86.95) (width 1.7) (layer "B.Cu") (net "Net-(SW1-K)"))
 (segment (start 135.9 75.89) (end 135.9 76.1) (width 0.2) (layer "B.Cu") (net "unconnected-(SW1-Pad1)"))
 (segment (start 135.55 75.75) (end 135.9 76.1) (width 0.2) (layer "B.Cu") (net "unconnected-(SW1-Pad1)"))
 (segment (start 129.025 78.485) (end 131.64 81.1) (width 1.7) (layer "B.Cu") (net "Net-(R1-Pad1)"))
 (segment (start 131.64 81.1) (end 135.9 81.1) (width 1.7) (layer "B.Cu") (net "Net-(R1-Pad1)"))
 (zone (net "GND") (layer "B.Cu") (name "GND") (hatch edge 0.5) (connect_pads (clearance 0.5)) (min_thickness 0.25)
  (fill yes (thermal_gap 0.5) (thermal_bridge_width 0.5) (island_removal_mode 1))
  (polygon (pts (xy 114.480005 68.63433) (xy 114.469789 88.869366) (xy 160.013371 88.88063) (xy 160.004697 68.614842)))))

